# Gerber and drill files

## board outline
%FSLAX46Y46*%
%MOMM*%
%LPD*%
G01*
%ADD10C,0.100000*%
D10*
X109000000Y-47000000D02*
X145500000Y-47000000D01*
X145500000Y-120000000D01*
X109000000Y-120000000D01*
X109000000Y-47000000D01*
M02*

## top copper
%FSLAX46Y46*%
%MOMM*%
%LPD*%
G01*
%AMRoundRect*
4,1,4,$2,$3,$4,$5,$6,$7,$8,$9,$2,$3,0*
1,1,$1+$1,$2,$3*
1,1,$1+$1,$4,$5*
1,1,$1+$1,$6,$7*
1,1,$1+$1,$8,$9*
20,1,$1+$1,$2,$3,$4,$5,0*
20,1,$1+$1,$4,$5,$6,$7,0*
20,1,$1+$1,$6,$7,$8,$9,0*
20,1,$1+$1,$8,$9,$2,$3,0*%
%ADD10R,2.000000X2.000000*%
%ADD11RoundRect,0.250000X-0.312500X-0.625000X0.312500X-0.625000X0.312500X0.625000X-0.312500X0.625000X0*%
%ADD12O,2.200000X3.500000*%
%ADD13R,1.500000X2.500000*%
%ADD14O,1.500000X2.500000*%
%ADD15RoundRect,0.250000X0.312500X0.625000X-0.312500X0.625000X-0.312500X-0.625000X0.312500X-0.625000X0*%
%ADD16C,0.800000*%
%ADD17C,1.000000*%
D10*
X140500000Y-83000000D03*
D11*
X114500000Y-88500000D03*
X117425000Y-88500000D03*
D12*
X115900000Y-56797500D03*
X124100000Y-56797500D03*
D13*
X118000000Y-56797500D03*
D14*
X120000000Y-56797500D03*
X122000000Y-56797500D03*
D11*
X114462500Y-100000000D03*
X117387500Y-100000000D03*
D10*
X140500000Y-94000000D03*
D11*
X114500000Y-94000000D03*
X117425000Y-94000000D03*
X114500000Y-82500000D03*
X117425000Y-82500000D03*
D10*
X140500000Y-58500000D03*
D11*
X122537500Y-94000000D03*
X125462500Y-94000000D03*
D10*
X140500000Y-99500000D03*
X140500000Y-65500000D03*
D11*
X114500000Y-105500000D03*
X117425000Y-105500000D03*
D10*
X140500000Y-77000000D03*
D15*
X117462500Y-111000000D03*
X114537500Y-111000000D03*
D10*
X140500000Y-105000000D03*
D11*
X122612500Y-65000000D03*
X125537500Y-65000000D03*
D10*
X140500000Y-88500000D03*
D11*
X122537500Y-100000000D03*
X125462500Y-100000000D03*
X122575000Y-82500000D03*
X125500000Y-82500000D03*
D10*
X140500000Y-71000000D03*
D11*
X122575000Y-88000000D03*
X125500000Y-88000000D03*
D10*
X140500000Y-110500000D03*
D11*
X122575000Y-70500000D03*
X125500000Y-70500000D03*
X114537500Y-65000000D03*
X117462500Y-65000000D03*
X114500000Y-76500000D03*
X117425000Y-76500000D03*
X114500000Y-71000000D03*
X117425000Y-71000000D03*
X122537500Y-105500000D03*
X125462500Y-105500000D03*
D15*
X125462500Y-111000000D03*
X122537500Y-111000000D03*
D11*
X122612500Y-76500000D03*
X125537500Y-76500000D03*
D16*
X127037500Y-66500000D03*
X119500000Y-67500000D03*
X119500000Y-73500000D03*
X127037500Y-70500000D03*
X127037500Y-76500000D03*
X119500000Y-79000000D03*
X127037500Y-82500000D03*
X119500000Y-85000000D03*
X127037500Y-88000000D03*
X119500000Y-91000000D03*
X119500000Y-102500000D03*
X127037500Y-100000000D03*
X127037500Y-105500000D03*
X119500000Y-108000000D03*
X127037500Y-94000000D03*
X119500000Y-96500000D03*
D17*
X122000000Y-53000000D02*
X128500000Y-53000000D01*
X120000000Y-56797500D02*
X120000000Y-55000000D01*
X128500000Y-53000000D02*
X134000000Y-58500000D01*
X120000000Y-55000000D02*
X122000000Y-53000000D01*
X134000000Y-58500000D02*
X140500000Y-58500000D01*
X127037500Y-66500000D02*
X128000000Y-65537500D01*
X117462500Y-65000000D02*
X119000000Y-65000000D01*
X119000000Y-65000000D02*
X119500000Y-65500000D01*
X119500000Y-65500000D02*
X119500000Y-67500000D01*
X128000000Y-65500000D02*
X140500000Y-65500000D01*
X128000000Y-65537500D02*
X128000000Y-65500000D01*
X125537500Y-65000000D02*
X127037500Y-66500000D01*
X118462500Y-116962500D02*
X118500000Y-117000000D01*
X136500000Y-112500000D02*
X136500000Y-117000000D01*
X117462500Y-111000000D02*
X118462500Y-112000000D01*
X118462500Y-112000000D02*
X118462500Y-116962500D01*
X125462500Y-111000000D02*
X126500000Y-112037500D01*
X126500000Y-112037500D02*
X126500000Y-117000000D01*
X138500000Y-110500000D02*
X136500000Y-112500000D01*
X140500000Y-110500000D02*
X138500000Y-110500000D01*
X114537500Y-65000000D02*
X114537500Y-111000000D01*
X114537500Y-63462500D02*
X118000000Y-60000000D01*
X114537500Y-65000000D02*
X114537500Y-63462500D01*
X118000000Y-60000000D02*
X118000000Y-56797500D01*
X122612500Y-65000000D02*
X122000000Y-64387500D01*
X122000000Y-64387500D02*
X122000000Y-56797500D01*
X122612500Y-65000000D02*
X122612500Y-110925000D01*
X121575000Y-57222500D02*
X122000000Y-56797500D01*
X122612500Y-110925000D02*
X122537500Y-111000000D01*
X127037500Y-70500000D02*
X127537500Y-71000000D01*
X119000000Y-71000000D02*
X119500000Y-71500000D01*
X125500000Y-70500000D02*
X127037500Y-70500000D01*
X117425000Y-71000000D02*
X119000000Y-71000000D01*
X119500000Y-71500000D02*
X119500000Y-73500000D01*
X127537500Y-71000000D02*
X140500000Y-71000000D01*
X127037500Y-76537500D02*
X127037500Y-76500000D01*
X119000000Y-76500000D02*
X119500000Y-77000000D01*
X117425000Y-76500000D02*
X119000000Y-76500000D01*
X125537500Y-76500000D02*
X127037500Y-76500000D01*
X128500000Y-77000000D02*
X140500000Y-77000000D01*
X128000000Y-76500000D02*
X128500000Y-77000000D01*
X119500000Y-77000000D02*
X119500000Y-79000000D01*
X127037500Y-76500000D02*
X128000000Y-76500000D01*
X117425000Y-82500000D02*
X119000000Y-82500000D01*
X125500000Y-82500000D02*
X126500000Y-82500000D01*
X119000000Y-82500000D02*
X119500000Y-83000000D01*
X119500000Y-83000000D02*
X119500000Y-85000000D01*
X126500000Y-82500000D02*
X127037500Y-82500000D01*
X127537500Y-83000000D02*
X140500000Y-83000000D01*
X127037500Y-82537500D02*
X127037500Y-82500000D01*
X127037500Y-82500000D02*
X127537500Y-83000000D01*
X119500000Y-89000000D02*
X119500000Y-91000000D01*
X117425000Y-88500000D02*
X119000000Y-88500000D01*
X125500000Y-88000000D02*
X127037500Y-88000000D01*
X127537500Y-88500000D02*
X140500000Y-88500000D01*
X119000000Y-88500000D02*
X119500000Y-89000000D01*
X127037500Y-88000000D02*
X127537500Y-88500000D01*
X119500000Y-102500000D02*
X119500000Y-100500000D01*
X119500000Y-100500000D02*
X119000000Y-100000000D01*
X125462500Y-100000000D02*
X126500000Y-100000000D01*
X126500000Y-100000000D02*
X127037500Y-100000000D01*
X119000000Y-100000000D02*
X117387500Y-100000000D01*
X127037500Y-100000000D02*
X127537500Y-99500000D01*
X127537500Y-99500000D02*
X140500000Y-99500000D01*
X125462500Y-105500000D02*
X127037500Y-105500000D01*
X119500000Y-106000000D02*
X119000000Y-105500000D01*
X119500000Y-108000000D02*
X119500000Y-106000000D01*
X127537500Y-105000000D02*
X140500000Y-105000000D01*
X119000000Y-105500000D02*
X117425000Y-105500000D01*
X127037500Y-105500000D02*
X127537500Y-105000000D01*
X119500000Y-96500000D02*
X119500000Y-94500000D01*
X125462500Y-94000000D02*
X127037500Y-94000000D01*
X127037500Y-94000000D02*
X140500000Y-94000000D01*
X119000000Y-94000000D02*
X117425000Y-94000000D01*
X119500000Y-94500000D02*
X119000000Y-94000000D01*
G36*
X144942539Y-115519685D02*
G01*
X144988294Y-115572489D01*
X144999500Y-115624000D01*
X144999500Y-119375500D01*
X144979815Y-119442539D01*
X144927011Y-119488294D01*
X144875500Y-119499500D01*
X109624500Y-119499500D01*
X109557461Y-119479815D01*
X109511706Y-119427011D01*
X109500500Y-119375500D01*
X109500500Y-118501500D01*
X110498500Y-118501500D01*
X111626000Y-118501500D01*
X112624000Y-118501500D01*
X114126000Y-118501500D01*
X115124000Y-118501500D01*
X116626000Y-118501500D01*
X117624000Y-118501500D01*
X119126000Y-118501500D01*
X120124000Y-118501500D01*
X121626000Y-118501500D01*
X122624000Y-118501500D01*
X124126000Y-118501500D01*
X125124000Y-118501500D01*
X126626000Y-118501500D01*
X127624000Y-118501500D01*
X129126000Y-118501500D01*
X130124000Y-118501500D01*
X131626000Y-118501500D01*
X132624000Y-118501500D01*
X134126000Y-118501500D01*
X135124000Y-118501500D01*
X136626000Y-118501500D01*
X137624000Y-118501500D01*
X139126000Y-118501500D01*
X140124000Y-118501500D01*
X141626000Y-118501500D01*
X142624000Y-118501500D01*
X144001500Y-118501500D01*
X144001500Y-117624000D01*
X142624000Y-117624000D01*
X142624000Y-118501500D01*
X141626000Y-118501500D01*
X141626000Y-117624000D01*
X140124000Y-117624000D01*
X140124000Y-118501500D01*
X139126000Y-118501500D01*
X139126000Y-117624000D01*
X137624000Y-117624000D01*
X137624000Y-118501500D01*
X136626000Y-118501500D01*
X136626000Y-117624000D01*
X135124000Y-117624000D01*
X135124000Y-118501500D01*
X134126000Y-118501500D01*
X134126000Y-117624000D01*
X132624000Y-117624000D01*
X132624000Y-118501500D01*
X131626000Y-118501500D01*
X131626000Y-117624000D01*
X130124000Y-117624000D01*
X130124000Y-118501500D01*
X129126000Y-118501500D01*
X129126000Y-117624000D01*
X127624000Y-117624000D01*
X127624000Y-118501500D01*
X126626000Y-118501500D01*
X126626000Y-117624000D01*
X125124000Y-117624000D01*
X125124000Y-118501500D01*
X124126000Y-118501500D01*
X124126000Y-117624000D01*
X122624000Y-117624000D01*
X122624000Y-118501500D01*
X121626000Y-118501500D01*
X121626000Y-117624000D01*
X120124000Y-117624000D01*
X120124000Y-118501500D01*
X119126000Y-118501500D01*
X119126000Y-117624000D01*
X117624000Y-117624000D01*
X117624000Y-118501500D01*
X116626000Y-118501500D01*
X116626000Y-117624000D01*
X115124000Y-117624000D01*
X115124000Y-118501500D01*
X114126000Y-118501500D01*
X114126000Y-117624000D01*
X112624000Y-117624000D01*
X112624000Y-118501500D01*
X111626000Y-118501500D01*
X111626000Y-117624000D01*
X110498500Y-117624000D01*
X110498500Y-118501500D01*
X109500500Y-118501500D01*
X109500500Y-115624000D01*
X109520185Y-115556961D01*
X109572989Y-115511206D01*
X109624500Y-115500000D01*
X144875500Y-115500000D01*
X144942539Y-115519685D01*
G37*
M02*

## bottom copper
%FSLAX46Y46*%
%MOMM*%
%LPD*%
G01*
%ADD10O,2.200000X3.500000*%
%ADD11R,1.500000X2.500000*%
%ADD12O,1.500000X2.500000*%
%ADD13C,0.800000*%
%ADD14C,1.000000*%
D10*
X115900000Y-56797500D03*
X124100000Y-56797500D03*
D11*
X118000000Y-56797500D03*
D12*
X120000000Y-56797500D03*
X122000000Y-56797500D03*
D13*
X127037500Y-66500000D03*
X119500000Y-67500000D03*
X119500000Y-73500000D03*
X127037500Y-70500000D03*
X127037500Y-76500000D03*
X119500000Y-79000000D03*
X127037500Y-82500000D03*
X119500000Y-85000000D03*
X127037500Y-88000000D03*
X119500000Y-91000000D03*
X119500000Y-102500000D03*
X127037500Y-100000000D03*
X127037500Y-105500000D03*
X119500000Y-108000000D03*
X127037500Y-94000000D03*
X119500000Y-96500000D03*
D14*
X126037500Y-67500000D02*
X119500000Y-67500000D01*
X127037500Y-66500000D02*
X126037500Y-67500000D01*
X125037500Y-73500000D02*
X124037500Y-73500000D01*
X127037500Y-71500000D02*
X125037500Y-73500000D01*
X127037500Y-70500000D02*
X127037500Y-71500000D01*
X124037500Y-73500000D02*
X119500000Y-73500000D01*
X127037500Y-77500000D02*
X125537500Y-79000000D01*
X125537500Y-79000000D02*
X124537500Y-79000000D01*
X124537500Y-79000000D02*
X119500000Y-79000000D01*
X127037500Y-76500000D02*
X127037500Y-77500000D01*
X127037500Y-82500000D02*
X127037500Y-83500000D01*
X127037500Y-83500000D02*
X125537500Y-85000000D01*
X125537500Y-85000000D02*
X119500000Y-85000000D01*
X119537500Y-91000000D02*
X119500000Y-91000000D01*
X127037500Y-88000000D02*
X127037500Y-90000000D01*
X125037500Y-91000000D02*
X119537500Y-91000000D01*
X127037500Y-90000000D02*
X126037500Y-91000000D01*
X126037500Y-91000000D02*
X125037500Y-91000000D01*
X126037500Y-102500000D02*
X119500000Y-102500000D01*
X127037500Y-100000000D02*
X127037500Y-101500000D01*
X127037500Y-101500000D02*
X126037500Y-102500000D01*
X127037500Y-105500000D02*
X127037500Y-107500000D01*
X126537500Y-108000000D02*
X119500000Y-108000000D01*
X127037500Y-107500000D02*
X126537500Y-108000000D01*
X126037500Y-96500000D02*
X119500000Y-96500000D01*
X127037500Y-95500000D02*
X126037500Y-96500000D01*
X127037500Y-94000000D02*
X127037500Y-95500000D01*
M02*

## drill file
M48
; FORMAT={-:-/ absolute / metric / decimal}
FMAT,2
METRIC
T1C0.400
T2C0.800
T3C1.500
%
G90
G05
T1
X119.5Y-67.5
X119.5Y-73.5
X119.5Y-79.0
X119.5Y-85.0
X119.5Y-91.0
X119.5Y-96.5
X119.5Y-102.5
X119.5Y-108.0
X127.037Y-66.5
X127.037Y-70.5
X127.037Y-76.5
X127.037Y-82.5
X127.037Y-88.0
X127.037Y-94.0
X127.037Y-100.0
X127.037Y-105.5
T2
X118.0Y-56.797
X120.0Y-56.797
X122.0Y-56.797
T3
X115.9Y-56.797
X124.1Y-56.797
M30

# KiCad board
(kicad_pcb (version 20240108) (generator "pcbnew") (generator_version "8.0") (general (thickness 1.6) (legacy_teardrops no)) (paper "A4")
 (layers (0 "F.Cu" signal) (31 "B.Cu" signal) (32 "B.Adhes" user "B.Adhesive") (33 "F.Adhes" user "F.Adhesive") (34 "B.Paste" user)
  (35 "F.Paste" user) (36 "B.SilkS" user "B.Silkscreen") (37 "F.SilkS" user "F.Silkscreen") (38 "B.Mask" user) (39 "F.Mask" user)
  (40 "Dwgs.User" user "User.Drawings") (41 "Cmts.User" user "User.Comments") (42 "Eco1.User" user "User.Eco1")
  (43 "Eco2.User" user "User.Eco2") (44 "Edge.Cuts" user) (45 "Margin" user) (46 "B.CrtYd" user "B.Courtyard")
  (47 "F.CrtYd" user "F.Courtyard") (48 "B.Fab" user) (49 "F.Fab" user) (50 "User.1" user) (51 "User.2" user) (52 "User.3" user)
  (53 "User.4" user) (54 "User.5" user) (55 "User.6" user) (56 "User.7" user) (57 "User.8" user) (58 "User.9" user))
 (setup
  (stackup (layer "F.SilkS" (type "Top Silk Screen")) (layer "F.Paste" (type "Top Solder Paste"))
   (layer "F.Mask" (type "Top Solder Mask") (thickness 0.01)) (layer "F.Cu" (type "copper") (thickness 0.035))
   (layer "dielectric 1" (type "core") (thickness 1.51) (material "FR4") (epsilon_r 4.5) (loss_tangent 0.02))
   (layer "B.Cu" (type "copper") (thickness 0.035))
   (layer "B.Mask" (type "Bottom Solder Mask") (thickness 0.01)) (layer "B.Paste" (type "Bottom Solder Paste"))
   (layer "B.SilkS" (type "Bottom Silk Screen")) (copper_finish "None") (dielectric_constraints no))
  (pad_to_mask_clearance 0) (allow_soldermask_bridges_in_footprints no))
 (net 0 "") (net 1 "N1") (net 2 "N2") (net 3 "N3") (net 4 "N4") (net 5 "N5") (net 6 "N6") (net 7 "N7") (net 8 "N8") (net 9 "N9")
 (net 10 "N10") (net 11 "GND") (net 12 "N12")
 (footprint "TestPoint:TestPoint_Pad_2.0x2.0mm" (layer "F.Cu") (at 140.5 83)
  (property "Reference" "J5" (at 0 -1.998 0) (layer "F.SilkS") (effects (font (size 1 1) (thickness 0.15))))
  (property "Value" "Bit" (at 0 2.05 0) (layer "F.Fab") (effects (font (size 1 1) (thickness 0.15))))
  (pad "1" smd rect (at 0 0) (size 2 2) (layers "F.Cu" "F.Mask") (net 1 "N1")))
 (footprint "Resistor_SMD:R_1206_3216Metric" (layer "F.Cu") (at 115.9625 88.5)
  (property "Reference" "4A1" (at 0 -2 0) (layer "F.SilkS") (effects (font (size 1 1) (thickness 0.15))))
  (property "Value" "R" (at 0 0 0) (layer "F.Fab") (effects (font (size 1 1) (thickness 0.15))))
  (pad "1" smd roundrect (at -1.4625 0) (size 1.125 1.75) (layers "F.Cu" "F.Paste" "F.Mask") (roundrect_rratio 0.222222) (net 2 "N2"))
  (pad "2" smd roundrect (at 1.4625 0) (size 1.125 1.75) (layers "F.Cu" "F.Paste" "F.Mask") (roundrect_rratio 0.222222) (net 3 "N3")))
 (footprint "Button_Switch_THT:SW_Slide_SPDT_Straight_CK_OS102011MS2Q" (layer "F.Cu") (at 118 56.7975)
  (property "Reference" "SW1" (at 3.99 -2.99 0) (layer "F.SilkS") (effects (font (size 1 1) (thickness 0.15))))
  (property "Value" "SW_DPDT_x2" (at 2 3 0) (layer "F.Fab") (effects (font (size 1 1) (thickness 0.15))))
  (pad "" thru_hole oval (at -2.1 0) (size 2.2 3.5) (drill 1.5) (layers "*.Cu" "*.Mask") (remove_unused_layers no))
  (pad "" thru_hole oval (at 6.1 0) (size 2.2 3.5) (drill 1.5) (layers "*.Cu" "*.Mask") (remove_unused_layers no))
  (pad "1" thru_hole rect (at 0 0) (size 1.5 2.5) (drill 0.8) (layers "*.Cu" "*.Mask") (remove_unused_layers no) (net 2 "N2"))
  (pad "2" thru_hole oval (at 2 0) (size 1.5 2.5) (drill 0.8) (layers "*.Cu" "*.Mask") (remove_unused_layers no) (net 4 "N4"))
  (pad "3" thru_hole oval (at 4 0) (size 1.5 2.5) (drill 0.8) (layers "*.Cu" "*.Mask") (remove_unused_layers no) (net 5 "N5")))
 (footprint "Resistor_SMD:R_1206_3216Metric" (layer "F.Cu") (at 115.925 100)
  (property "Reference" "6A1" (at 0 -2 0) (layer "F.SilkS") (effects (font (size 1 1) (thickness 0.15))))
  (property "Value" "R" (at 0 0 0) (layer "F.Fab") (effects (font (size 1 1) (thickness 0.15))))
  (pad "1" smd roundrect (at -1.4625 0) (size 1.125 1.75) (layers "F.Cu" "F.Paste" "F.Mask") (roundrect_rratio 0.222222) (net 2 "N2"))
  (pad "2" smd roundrect (at 1.4625 0) (size 1.125 1.75) (layers "F.Cu" "F.Paste" "F.Mask") (roundrect_rratio 0.222222) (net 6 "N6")))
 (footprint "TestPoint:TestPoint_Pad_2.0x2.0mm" (layer "F.Cu") (at 140.5 94)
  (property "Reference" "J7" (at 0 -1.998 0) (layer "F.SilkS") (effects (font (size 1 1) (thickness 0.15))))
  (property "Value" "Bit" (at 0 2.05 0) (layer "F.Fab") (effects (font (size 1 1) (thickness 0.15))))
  (pad "1" smd rect (at 0 0) (size 2 2) (layers "F.Cu" "F.Mask") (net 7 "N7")))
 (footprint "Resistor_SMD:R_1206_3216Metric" (layer "F.Cu") (at 115.9625 94)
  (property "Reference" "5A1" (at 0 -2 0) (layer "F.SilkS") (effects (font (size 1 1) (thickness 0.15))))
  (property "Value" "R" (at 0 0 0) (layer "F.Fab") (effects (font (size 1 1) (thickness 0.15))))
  (pad "1" smd roundrect (at -1.4625 0) (size 1.125 1.75) (layers "F.Cu" "F.Paste" "F.Mask") (roundrect_rratio 0.222222) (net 2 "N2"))
  (pad "2" smd roundrect (at 1.4625 0) (size 1.125 1.75) (layers "F.Cu" "F.Paste" "F.Mask") (roundrect_rratio 0.222222) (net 7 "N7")))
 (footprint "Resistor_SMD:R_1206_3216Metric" (layer "F.Cu") (at 115.9625 82.5)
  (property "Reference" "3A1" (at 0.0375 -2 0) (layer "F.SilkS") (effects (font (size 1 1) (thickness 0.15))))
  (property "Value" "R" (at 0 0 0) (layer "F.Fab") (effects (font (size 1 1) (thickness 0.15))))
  (pad "1" smd roundrect (at -1.4625 0) (size 1.125 1.75) (layers "F.Cu" "F.Paste" "F.Mask") (roundrect_rratio 0.222222) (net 2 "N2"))
  (pad "2" smd roundrect (at 1.4625 0) (size 1.125 1.75) (layers "F.Cu" "F.Paste" "F.Mask") (roundrect_rratio 0.222222) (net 1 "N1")))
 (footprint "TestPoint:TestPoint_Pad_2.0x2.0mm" (layer "F.Cu") (at 140.5 58.5)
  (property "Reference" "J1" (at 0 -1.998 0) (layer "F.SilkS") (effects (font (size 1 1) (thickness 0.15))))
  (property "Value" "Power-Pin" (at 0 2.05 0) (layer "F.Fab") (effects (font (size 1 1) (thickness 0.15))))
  (pad "1" smd rect (at 0 0) (size 2 2) (layers "F.Cu" "F.Mask") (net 4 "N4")))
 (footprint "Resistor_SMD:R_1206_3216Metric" (layer "F.Cu") (at 124 94)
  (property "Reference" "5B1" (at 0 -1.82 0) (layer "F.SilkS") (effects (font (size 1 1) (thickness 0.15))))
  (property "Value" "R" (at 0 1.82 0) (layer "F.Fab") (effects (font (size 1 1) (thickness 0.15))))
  (pad "1" smd roundrect (at -1.4625 0) (size 1.125 1.75) (layers "F.Cu" "F.Paste" "F.Mask") (roundrect_rratio 0.222222) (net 5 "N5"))
  (pad "2" smd roundrect (at 1.4625 0) (size 1.125 1.75) (layers "F.Cu" "F.Paste" "F.Mask") (roundrect_rratio 0.222222) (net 7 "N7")))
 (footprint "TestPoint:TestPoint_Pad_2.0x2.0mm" (layer "F.Cu") (at 140.5 99.5)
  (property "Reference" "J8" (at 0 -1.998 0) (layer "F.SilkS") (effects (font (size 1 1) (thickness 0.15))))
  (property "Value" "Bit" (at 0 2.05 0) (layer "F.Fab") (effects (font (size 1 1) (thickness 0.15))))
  (pad "1" smd rect (at 0 0) (size 2 2) (layers "F.Cu" "F.Mask") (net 6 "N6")))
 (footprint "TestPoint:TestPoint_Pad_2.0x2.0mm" (layer "F.Cu") (at 140.5 65.5)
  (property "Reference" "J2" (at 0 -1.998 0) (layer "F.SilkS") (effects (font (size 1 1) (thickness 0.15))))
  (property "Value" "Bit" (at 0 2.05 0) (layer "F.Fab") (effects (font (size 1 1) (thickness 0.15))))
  (pad "1" smd rect (at 0 0) (size 2 2) (layers "F.Cu" "F.Mask") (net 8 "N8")))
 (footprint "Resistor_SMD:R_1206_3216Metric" (layer "F.Cu") (at 115.9625 105.5)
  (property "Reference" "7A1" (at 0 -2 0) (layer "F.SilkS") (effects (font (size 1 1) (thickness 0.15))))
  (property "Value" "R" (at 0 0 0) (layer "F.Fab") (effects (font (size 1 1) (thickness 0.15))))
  (pad "1" smd roundrect (at -1.4625 0) (size 1.125 1.75) (layers "F.Cu" "F.Paste" "F.Mask") (roundrect_rratio 0.222222) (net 2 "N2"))
  (pad "2" smd roundrect (at 1.4625 0) (size 1.125 1.75) (layers "F.Cu" "F.Paste" "F.Mask") (roundrect_rratio 0.222222) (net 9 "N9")))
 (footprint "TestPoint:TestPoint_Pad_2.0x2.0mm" (layer "F.Cu") (at 140.5 77)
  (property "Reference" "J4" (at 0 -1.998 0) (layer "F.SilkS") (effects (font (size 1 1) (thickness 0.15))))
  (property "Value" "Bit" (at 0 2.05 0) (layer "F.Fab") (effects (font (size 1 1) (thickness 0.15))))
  (pad "1" smd rect (at 0 0) (size 2 2) (layers "F.Cu" "F.Mask") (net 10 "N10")))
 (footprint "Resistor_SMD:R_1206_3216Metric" (layer "F.Cu") (at 116 111 180)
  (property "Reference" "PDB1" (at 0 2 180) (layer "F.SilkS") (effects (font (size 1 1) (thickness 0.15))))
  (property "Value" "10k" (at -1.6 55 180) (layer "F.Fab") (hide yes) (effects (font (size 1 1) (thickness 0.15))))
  (pad "1" smd roundrect (at -1.4625 0 180) (size 1.125 1.75) (layers "F.Cu" "F.Paste" "F.Mask") (roundrect_rratio 0.222222) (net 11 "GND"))
  (pad "2" smd roundrect (at 1.4625 0 180) (size 1.125 1.75) (layers "F.Cu" "F.Paste" "F.Mask") (roundrect_rratio 0.222222) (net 2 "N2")))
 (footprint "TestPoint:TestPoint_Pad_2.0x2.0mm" (layer "F.Cu") (at 140.5 105)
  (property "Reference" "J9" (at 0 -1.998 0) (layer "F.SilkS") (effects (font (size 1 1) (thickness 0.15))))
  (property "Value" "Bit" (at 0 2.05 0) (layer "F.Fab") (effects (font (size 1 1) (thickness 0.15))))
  (pad "1" smd rect (at 0 0) (size 2 2) (layers "F.Cu" "F.Mask") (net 9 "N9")))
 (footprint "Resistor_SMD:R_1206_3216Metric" (layer "F.Cu") (at 124.075 65)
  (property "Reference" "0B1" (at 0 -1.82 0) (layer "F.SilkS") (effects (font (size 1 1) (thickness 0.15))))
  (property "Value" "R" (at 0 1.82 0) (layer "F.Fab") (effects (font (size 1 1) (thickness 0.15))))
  (pad "1" smd roundrect (at -1.4625 0) (size 1.125 1.75) (layers "F.Cu" "F.Paste" "F.Mask") (roundrect_rratio 0.222222) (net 5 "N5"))
  (pad "2" smd roundrect (at 1.4625 0) (size 1.125 1.75) (layers "F.Cu" "F.Paste" "F.Mask") (roundrect_rratio 0.222222) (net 8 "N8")))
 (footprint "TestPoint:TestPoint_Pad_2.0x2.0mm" (layer "F.Cu") (at 140.5 88.5)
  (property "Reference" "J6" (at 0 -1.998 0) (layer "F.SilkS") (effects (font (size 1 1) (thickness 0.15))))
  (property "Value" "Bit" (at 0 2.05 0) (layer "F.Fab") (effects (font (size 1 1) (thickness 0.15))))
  (pad "1" smd rect (at 0 0) (size 2 2) (layers "F.Cu" "F.Mask") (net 3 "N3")))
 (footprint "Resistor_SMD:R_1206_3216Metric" (layer "F.Cu") (at 124 100)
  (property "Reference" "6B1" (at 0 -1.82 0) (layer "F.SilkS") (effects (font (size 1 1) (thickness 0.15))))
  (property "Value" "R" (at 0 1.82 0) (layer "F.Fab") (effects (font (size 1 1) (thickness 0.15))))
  (pad "1" smd roundrect (at -1.4625 0) (size 1.125 1.75) (layers "F.Cu" "F.Paste" "F.Mask") (roundrect_rratio 0.222222) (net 5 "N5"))
  (pad "2" smd roundrect (at 1.4625 0) (size 1.125 1.75) (layers "F.Cu" "F.Paste" "F.Mask") (roundrect_rratio 0.222222) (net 6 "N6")))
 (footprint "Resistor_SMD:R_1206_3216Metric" (layer "F.Cu") (at 124.0375 82.5)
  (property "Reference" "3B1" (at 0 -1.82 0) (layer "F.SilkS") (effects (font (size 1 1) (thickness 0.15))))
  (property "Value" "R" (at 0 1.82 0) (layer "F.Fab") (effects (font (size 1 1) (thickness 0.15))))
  (pad "1" smd roundrect (at -1.4625 0) (size 1.125 1.75) (layers "F.Cu" "F.Paste" "F.Mask") (roundrect_rratio 0.222222) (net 5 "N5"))
  (pad "2" smd roundrect (at 1.4625 0) (size 1.125 1.75) (layers "F.Cu" "F.Paste" "F.Mask") (roundrect_rratio 0.222222) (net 1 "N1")))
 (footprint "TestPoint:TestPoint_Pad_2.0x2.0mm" (layer "F.Cu") (at 140.5 71)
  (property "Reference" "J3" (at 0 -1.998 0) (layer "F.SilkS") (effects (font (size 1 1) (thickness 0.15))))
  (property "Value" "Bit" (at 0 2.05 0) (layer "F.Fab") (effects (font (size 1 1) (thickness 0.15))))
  (pad "1" smd rect (at 0 0) (size 2 2) (layers "F.Cu" "F.Mask") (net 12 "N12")))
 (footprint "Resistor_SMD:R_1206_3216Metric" (layer "F.Cu") (at 124.0375 88)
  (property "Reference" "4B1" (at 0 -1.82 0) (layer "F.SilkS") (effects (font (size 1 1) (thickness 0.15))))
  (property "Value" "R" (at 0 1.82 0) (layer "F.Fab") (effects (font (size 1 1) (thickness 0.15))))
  (pad "1" smd roundrect (at -1.4625 0) (size 1.125 1.75) (layers "F.Cu" "F.Paste" "F.Mask") (roundrect_rratio 0.222222) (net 5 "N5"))
  (pad "2" smd roundrect (at 1.4625 0) (size 1.125 1.75) (layers "F.Cu" "F.Paste" "F.Mask") (roundrect_rratio 0.222222) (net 3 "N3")))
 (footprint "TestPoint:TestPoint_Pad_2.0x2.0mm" (layer "F.Cu") (at 140.5 110.5)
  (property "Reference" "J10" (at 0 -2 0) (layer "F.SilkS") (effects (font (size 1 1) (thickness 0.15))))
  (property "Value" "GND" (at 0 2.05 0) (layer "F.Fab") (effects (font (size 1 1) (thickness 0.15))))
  (pad "1" smd rect (at 0 0) (size 2 2) (layers "F.Cu" "F.Mask") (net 11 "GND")))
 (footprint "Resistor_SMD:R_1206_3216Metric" (layer "F.Cu") (at 124.0375 70.5)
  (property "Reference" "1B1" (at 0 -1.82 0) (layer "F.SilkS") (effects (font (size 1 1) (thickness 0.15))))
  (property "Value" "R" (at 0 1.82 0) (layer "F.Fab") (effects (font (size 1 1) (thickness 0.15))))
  (pad "1" smd roundrect (at -1.4625 0) (size 1.125 1.75) (layers "F.Cu" "F.Paste" "F.Mask") (roundrect_rratio 0.222222) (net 5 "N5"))
  (pad "2" smd roundrect (at 1.4625 0) (size 1.125 1.75) (layers "F.Cu" "F.Paste" "F.Mask") (roundrect_rratio 0.222222) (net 12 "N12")))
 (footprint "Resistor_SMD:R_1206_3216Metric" (layer "F.Cu") (at 116 65)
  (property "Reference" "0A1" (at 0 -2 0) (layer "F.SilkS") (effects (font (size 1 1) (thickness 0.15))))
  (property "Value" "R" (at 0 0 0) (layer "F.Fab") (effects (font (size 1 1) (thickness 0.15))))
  (pad "1" smd roundrect (at -1.4625 0) (size 1.125 1.75) (layers "F.Cu" "F.Paste" "F.Mask") (roundrect_rratio 0.222222) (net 2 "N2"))
  (pad "2" smd roundrect (at 1.4625 0) (size 1.125 1.75) (layers "F.Cu" "F.Paste" "F.Mask") (roundrect_rratio 0.222222) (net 8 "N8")))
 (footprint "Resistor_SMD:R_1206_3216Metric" (layer "F.Cu") (at 115.9625 76.5)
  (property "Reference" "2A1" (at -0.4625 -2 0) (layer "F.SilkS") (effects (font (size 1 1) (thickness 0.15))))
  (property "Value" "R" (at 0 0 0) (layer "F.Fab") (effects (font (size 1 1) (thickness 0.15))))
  (pad "1" smd roundrect (at -1.4625 0) (size 1.125 1.75) (layers "F.Cu" "F.Paste" "F.Mask") (roundrect_rratio 0.222222) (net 2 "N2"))
  (pad "2" smd roundrect (at 1.4625 0) (size 1.125 1.75) (layers "F.Cu" "F.Paste" "F.Mask") (roundrect_rratio 0.222222) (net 10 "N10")))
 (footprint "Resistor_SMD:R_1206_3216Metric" (layer "F.Cu") (at 115.9625 71)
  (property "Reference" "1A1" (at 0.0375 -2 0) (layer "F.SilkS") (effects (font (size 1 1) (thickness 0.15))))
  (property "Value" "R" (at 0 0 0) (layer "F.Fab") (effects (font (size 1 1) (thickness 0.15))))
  (pad "1" smd roundrect (at -1.4625 0) (size 1.125 1.75) (layers "F.Cu" "F.Paste" "F.Mask") (roundrect_rratio 0.222222) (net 2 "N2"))
  (pad "2" smd roundrect (at 1.4625 0) (size 1.125 1.75) (layers "F.Cu" "F.Paste" "F.Mask") (roundrect_rratio 0.222222) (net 12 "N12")))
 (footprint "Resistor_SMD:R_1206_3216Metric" (layer "F.Cu") (at 124 105.5)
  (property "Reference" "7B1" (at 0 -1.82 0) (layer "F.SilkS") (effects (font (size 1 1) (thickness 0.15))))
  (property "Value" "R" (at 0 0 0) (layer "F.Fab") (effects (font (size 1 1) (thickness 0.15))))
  (pad "1" smd roundrect (at -1.4625 0) (size 1.125 1.75) (layers "F.Cu" "F.Paste" "F.Mask") (roundrect_rratio 0.222222) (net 5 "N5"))
  (pad "2" smd roundrect (at 1.4625 0) (size 1.125 1.75) (layers "F.Cu" "F.Paste" "F.Mask") (roundrect_rratio 0.222222) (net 9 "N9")))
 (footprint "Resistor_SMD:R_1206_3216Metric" (layer "F.Cu") (at 124 111 180)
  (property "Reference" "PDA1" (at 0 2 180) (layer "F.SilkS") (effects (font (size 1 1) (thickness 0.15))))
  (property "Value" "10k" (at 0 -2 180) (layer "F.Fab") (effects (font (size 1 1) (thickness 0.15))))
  (pad "1" smd roundrect (at -1.4625 0 180) (size 1.125 1.75) (layers "F.Cu" "F.Paste" "F.Mask") (roundrect_rratio 0.222222) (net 11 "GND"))
  (pad "2" smd roundrect (at 1.4625 0 180) (size 1.125 1.75) (layers "F.Cu" "F.Paste" "F.Mask") (roundrect_rratio 0.222222) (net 5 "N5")))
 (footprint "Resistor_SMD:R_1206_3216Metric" (layer "F.Cu") (at 124.075 76.5)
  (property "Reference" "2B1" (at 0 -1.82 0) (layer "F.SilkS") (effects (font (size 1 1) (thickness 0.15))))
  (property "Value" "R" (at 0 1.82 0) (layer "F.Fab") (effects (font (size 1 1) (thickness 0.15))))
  (pad "1" smd roundrect (at -1.4625 0) (size 1.125 1.75) (layers "F.Cu" "F.Paste" "F.Mask") (roundrect_rratio 0.222222) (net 5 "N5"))
  (pad "2" smd roundrect (at 1.4625 0) (size 1.125 1.75) (layers "F.Cu" "F.Paste" "F.Mask") (roundrect_rratio 0.222222) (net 10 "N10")))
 (gr_rect (start 109 47) (end 145.5 120) (stroke (width 0.1) (type default)) (fill none) (layer "Edge.Cuts"))
 (segment (start 122 53) (end 128.5 53) (width 1) (layer "F.Cu") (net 4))
 (segment (start 120 56.7975) (end 120 55) (width 1) (layer "F.Cu") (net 4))
 (segment (start 128.5 53) (end 134 58.5) (width 1) (layer "F.Cu") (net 4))
 (segment (start 120 55) (end 122 53) (width 1) (layer "F.Cu") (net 4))
 (segment (start 134 58.5) (end 140.5 58.5) (width 1) (layer "F.Cu") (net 4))
 (segment (start 127.0375 66.5) (end 128 65.5375) (width 1) (layer "F.Cu") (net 8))
 (segment (start 117.4625 65) (end 119 65) (width 1) (layer "F.Cu") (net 8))
 (segment (start 119 65) (end 119.5 65.5) (width 1) (layer "F.Cu") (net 8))
 (segment (start 119.5 65.5) (end 119.5 67.5) (width 1) (layer "F.Cu") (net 8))
 (segment (start 128 65.5) (end 140.5 65.5) (width 1) (layer "F.Cu") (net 8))
 (segment (start 128 65.5375) (end 128 65.5) (width 1) (layer "F.Cu") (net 8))
 (segment (start 125.5375 65) (end 127.0375 66.5) (width 1) (layer "F.Cu") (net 8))
 (via (at 127.0375 66.5) (size 0.8) (drill 0.4) (layers "F.Cu" "B.Cu") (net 8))
 (via (at 119.5 67.5) (size 0.8) (drill 0.4) (layers "F.Cu" "B.Cu") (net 8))
 (segment (start 126.0375 67.5) (end 119.5 67.5) (width 1) (layer "B.Cu") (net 8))
 (segment (start 127.0375 66.5) (end 126.0375 67.5) (width 1) (layer "B.Cu") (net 8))
 (segment (start 118.4625 116.9625) (end 118.5 117) (width 1) (layer "F.Cu") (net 11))
 (segment (start 136.5 112.5) (end 136.5 117) (width 1) (layer "F.Cu") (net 11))
 (segment (start 117.4625 111) (end 118.4625 112) (width 1) (layer "F.Cu") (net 11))
 (segment (start 118.4625 112) (end 118.4625 116.9625) (width 1) (layer "F.Cu") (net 11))
 (segment (start 125.4625 111) (end 126.5 112.0375) (width 1) (layer "F.Cu") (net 11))
 (segment (start 126.5 112.0375) (end 126.5 117) (width 1) (layer "F.Cu") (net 11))
 (segment (start 138.5 110.5) (end 136.5 112.5) (width 1) (layer "F.Cu") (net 11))
 (segment (start 140.5 110.5) (end 138.5 110.5) (width 1) (layer "F.Cu") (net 11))
 (segment (start 114.5375 65) (end 114.5375 111) (width 1) (layer "F.Cu") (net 2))
 (segment (start 114.5375 63.4625) (end 118 60) (width 1) (layer "F.Cu") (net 2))
 (segment (start 114.5375 65) (end 114.5375 63.4625) (width 1) (layer "F.Cu") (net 2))
 (segment (start 118 60) (end 118 56.7975) (width 1) (layer "F.Cu") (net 2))
 (segment (start 122.6125 65) (end 122 64.3875) (width 1) (layer "F.Cu") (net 5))
 (segment (start 122 64.3875) (end 122 56.7975) (width 1) (layer "F.Cu") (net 5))
 (segment (start 122.6125 65) (end 122.6125 110.925) (width 1) (layer "F.Cu") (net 5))
 (segment (start 121.575 57.2225) (end 122 56.7975) (width 1) (layer "F.Cu") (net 5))
 (segment (start 122.6125 110.925) (end 122.5375 111) (width 1) (layer "F.Cu") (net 5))
 (segment (start 127.0375 70.5) (end 127.5375 71) (width 1) (layer "F.Cu") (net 12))
 (segment (start 119 71) (end 119.5 71.5) (width 1) (layer "F.Cu") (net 12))
 (segment (start 125.5 70.5) (end 127.0375 70.5) (width 1) (layer "F.Cu") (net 12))
 (segment (start 117.425 71) (end 119 71) (width 1) (layer "F.Cu") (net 12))
 (segment (start 119.5 71.5) (end 119.5 73.5) (width 1) (layer "F.Cu") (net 12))
 (segment (start 127.5375 71) (end 140.5 71) (width 1) (layer "F.Cu") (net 12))
 (via (at 119.5 73.5) (size 0.8) (drill 0.4) (layers "F.Cu" "B.Cu") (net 12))
 (via (at 127.0375 70.5) (size 0.8) (drill 0.4) (layers "F.Cu" "B.Cu") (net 12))
 (segment (start 125.0375 73.5) (end 124.0375 73.5) (width 1) (layer "B.Cu") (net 12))
 (segment (start 127.0375 71.5) (end 125.0375 73.5) (width 1) (layer "B.Cu") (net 12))
 (segment (start 127.0375 70.5) (end 127.0375 71.5) (width 1) (layer "B.Cu") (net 12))
 (segment (start 124.0375 73.5) (end 119.5 73.5) (width 1) (layer "B.Cu") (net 12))
 (segment (start 127.0375 76.5375) (end 127.0375 76.5) (width 1) (layer "F.Cu") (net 10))
 (segment (start 119 76.5) (end 119.5 77) (width 1) (layer "F.Cu") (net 10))
 (segment (start 117.425 76.5) (end 119 76.5) (width 1) (layer "F.Cu") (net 10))
 (segment (start 125.5375 76.5) (end 127.0375 76.5) (width 1) (layer "F.Cu") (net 10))
 (segment (start 128.5 77) (end 140.5 77) (width 1) (layer "F.Cu") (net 10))
 (segment (start 128 76.5) (end 128.5 77) (width 1) (layer "F.Cu") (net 10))
 (segment (start 119.5 77) (end 119.5 79) (width 1) (layer "F.Cu") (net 10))
 (segment (start 127.0375 76.5) (end 128 76.5) (width 1) (layer "F.Cu") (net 10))
 (via (at 127.0375 76.5) (size 0.8) (drill 0.4) (layers "F.Cu" "B.Cu") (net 10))
 (via (at 119.5 79) (size 0.8) (drill 0.4) (layers "F.Cu" "B.Cu") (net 10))
 (segment (start 127.0375 77.5) (end 125.5375 79) (width 1) (layer "B.Cu") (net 10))
 (segment (start 125.5375 79) (end 124.5375 79) (width 1) (layer "B.Cu") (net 10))
 (segment (start 124.5375 79) (end 119.5 79) (width 1) (layer "B.Cu") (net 10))
 (segment (start 127.0375 76.5) (end 127.0375 77.5) (width 1) (layer "B.Cu") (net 10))
 (segment (start 117.425 82.5) (end 119 82.5) (width 1) (layer "F.Cu") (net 1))
 (segment (start 125.5 82.5) (end 126.5 82.5) (width 1) (layer "F.Cu") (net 1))
 (segment (start 119 82.5) (end 119.5 83) (width 1) (layer "F.Cu") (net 1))
 (segment (start 119.5 83) (end 119.5 85) (width 1) (layer "F.Cu") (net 1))
 (segment (start 126.5 82.5) (end 127.0375 82.5) (width 1) (layer "F.Cu") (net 1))
 (segment (start 127.5375 83) (end 140.5 83) (width 1) (layer "F.Cu") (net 1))
 (segment (start 127.0375 82.5375) (end 127.0375 82.5) (width 1) (layer "F.Cu") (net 1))
 (segment (start 127.0375 82.5) (end 127.5375 83) (width 1) (layer "F.Cu") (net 1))
 (via (at 127.0375 82.5) (size 0.8) (drill 0.4) (layers "F.Cu" "B.Cu") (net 1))
 (via (at 119.5 85) (size 0.8) (drill 0.4) (layers "F.Cu" "B.Cu") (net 1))
 (segment (start 127.0375 82.5) (end 127.0375 83.5) (width 1) (layer "B.Cu") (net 1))
 (segment (start 127.0375 83.5) (end 125.5375 85) (width 1) (layer "B.Cu") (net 1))
 (segment (start 125.5375 85) (end 119.5 85) (width 1) (layer "B.Cu") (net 1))
 (segment (start 119.5 89) (end 119.5 91) (width 1) (layer "F.Cu") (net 3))
 (segment (start 117.425 88.5) (end 119 88.5) (width 1) (layer "F.Cu") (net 3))
 (segment (start 125.5 88) (end 127.0375 88) (width 1) (layer "F.Cu") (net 3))
 (segment (start 127.5375 88.5) (end 140.5 88.5) (width 1) (layer "F.Cu") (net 3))
 (segment (start 119 88.5) (end 119.5 89) (width 1) (layer "F.Cu") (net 3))
 (segment (start 127.0375 88) (end 127.5375 88.5) (width 1) (layer "F.Cu") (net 3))
 (via (at 127.0375 88) (size 0.8) (drill 0.4) (layers "F.Cu" "B.Cu") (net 3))
 (via (at 119.5 91) (size 0.8) (drill 0.4) (layers "F.Cu" "B.Cu") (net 3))
 (segment (start 119.5375 91) (end 119.5 91) (width 1) (layer "B.Cu") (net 3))
 (segment (start 127.0375 88) (end 127.0375 90) (width 1) (layer "B.Cu") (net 3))
 (segment (start 125.0375 91) (end 119.5375 91) (width 1) (layer "B.Cu") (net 3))
 (segment (start 127.0375 90) (end 126.0375 91) (width 1) (layer "B.Cu") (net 3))
 (segment (start 126.0375 91) (end 125.0375 91) (width 1) (layer "B.Cu") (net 3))
 (segment (start 119.5 102.5) (end 119.5 100.5) (width 1) (layer "F.Cu") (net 6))
 (segment (start 119.5 100.5) (end 119 100) (width 1) (layer "F.Cu") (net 6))
 (segment (start 125.4625 100) (end 126.5 100) (width 1) (layer "F.Cu") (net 6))
 (segment (start 126.5 100) (end 127.0375 100) (width 1) (layer "F.Cu") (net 6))
 (segment (start 119 100) (end 117.3875 100) (width 1) (layer "F.Cu") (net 6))
 (segment (start 127.0375 100) (end 127.5375 99.5) (width 1) (layer "F.Cu") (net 6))
 (segment (start 127.5375 99.5) (end 140.5 99.5) (width 1) (layer "F.Cu") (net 6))
 (via (at 119.5 102.5) (size 0.8) (drill 0.4) (layers "F.Cu" "B.Cu") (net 6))
 (via (at 127.0375 100) (size 0.8) (drill 0.4) (layers "F.Cu" "B.Cu") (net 6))
 (segment (start 126.0375 102.5) (end 119.5 102.5) (width 1) (layer "B.Cu") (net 6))
 (segment (start 127.0375 100) (end 127.0375 101.5) (width 1) (layer "B.Cu") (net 6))
 (segment (start 127.0375 101.5) (end 126.0375 102.5) (width 1) (layer "B.Cu") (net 6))
 (segment (start 125.4625 105.5) (end 127.0375 105.5) (width 1) (layer "F.Cu") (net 9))
 (segment (start 119.5 106) (end 119 105.5) (width 1) (layer "F.Cu") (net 9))
 (segment (start 119.5 108) (end 119.5 106) (width 1) (layer "F.Cu") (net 9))
 (segment (start 127.5375 105) (end 140.5 105) (width 1) (layer "F.Cu") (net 9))
 (segment (start 119 105.5) (end 117.425 105.5) (width 1) (layer "F.Cu") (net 9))
 (segment (start 127.0375 105.5) (end 127.5375 105) (width 1) (layer "F.Cu") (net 9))
 (via (at 127.0375 105.5) (size 0.8) (drill 0.4) (layers "F.Cu" "B.Cu") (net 9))
 (via (at 119.5 108) (size 0.8) (drill 0.4) (layers "F.Cu" "B.Cu") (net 9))
 (segment (start 127.0375 105.5) (end 127.0375 107.5) (width 1) (layer "B.Cu") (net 9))
 (segment (start 126.5375 108) (end 119.5 108) (width 1) (layer "B.Cu") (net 9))
 (segment (start 127.0375 107.5) (end 126.5375 108) (width 1) (layer "B.Cu") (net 9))
 (segment (start 119.5 96.5) (end 119.5 94.5) (width 1) (layer "F.Cu") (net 7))
 (segment (start 125.4625 94) (end 127.0375 94) (width 1) (layer "F.Cu") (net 7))
 (segment (start 127.0375 94) (end 140.5 94) (width 1) (layer "F.Cu") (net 7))
 (segment (start 119 94) (end 117.425 94) (width 1) (layer "F.Cu") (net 7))
 (segment (start 119.5 94.5) (end 119 94) (width 1) (layer "F.Cu") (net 7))
 (via (at 127.0375 94) (size 0.8) (drill 0.4) (layers "F.Cu" "B.Cu") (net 7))
 (via (at 119.5 96.5) (size 0.8) (drill 0.4) (layers "F.Cu" "B.Cu") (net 7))
 (segment (start 126.0375 96.5) (end 119.5 96.5) (width 1) (layer "B.Cu") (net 7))
 (segment (start 127.0375 95.5) (end 126.0375 96.5) (width 1) (layer "B.Cu") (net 7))
 (segment (start 127.0375 94) (end 127.0375 95.5) (width 1) (layer "B.Cu") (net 7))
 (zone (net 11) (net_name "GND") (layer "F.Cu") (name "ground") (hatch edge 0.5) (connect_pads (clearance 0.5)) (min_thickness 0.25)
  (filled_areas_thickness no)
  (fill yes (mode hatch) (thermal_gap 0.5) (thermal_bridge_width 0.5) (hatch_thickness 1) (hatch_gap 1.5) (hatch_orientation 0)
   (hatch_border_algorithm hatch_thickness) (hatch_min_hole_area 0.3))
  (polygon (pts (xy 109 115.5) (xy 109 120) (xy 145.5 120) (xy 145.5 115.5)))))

